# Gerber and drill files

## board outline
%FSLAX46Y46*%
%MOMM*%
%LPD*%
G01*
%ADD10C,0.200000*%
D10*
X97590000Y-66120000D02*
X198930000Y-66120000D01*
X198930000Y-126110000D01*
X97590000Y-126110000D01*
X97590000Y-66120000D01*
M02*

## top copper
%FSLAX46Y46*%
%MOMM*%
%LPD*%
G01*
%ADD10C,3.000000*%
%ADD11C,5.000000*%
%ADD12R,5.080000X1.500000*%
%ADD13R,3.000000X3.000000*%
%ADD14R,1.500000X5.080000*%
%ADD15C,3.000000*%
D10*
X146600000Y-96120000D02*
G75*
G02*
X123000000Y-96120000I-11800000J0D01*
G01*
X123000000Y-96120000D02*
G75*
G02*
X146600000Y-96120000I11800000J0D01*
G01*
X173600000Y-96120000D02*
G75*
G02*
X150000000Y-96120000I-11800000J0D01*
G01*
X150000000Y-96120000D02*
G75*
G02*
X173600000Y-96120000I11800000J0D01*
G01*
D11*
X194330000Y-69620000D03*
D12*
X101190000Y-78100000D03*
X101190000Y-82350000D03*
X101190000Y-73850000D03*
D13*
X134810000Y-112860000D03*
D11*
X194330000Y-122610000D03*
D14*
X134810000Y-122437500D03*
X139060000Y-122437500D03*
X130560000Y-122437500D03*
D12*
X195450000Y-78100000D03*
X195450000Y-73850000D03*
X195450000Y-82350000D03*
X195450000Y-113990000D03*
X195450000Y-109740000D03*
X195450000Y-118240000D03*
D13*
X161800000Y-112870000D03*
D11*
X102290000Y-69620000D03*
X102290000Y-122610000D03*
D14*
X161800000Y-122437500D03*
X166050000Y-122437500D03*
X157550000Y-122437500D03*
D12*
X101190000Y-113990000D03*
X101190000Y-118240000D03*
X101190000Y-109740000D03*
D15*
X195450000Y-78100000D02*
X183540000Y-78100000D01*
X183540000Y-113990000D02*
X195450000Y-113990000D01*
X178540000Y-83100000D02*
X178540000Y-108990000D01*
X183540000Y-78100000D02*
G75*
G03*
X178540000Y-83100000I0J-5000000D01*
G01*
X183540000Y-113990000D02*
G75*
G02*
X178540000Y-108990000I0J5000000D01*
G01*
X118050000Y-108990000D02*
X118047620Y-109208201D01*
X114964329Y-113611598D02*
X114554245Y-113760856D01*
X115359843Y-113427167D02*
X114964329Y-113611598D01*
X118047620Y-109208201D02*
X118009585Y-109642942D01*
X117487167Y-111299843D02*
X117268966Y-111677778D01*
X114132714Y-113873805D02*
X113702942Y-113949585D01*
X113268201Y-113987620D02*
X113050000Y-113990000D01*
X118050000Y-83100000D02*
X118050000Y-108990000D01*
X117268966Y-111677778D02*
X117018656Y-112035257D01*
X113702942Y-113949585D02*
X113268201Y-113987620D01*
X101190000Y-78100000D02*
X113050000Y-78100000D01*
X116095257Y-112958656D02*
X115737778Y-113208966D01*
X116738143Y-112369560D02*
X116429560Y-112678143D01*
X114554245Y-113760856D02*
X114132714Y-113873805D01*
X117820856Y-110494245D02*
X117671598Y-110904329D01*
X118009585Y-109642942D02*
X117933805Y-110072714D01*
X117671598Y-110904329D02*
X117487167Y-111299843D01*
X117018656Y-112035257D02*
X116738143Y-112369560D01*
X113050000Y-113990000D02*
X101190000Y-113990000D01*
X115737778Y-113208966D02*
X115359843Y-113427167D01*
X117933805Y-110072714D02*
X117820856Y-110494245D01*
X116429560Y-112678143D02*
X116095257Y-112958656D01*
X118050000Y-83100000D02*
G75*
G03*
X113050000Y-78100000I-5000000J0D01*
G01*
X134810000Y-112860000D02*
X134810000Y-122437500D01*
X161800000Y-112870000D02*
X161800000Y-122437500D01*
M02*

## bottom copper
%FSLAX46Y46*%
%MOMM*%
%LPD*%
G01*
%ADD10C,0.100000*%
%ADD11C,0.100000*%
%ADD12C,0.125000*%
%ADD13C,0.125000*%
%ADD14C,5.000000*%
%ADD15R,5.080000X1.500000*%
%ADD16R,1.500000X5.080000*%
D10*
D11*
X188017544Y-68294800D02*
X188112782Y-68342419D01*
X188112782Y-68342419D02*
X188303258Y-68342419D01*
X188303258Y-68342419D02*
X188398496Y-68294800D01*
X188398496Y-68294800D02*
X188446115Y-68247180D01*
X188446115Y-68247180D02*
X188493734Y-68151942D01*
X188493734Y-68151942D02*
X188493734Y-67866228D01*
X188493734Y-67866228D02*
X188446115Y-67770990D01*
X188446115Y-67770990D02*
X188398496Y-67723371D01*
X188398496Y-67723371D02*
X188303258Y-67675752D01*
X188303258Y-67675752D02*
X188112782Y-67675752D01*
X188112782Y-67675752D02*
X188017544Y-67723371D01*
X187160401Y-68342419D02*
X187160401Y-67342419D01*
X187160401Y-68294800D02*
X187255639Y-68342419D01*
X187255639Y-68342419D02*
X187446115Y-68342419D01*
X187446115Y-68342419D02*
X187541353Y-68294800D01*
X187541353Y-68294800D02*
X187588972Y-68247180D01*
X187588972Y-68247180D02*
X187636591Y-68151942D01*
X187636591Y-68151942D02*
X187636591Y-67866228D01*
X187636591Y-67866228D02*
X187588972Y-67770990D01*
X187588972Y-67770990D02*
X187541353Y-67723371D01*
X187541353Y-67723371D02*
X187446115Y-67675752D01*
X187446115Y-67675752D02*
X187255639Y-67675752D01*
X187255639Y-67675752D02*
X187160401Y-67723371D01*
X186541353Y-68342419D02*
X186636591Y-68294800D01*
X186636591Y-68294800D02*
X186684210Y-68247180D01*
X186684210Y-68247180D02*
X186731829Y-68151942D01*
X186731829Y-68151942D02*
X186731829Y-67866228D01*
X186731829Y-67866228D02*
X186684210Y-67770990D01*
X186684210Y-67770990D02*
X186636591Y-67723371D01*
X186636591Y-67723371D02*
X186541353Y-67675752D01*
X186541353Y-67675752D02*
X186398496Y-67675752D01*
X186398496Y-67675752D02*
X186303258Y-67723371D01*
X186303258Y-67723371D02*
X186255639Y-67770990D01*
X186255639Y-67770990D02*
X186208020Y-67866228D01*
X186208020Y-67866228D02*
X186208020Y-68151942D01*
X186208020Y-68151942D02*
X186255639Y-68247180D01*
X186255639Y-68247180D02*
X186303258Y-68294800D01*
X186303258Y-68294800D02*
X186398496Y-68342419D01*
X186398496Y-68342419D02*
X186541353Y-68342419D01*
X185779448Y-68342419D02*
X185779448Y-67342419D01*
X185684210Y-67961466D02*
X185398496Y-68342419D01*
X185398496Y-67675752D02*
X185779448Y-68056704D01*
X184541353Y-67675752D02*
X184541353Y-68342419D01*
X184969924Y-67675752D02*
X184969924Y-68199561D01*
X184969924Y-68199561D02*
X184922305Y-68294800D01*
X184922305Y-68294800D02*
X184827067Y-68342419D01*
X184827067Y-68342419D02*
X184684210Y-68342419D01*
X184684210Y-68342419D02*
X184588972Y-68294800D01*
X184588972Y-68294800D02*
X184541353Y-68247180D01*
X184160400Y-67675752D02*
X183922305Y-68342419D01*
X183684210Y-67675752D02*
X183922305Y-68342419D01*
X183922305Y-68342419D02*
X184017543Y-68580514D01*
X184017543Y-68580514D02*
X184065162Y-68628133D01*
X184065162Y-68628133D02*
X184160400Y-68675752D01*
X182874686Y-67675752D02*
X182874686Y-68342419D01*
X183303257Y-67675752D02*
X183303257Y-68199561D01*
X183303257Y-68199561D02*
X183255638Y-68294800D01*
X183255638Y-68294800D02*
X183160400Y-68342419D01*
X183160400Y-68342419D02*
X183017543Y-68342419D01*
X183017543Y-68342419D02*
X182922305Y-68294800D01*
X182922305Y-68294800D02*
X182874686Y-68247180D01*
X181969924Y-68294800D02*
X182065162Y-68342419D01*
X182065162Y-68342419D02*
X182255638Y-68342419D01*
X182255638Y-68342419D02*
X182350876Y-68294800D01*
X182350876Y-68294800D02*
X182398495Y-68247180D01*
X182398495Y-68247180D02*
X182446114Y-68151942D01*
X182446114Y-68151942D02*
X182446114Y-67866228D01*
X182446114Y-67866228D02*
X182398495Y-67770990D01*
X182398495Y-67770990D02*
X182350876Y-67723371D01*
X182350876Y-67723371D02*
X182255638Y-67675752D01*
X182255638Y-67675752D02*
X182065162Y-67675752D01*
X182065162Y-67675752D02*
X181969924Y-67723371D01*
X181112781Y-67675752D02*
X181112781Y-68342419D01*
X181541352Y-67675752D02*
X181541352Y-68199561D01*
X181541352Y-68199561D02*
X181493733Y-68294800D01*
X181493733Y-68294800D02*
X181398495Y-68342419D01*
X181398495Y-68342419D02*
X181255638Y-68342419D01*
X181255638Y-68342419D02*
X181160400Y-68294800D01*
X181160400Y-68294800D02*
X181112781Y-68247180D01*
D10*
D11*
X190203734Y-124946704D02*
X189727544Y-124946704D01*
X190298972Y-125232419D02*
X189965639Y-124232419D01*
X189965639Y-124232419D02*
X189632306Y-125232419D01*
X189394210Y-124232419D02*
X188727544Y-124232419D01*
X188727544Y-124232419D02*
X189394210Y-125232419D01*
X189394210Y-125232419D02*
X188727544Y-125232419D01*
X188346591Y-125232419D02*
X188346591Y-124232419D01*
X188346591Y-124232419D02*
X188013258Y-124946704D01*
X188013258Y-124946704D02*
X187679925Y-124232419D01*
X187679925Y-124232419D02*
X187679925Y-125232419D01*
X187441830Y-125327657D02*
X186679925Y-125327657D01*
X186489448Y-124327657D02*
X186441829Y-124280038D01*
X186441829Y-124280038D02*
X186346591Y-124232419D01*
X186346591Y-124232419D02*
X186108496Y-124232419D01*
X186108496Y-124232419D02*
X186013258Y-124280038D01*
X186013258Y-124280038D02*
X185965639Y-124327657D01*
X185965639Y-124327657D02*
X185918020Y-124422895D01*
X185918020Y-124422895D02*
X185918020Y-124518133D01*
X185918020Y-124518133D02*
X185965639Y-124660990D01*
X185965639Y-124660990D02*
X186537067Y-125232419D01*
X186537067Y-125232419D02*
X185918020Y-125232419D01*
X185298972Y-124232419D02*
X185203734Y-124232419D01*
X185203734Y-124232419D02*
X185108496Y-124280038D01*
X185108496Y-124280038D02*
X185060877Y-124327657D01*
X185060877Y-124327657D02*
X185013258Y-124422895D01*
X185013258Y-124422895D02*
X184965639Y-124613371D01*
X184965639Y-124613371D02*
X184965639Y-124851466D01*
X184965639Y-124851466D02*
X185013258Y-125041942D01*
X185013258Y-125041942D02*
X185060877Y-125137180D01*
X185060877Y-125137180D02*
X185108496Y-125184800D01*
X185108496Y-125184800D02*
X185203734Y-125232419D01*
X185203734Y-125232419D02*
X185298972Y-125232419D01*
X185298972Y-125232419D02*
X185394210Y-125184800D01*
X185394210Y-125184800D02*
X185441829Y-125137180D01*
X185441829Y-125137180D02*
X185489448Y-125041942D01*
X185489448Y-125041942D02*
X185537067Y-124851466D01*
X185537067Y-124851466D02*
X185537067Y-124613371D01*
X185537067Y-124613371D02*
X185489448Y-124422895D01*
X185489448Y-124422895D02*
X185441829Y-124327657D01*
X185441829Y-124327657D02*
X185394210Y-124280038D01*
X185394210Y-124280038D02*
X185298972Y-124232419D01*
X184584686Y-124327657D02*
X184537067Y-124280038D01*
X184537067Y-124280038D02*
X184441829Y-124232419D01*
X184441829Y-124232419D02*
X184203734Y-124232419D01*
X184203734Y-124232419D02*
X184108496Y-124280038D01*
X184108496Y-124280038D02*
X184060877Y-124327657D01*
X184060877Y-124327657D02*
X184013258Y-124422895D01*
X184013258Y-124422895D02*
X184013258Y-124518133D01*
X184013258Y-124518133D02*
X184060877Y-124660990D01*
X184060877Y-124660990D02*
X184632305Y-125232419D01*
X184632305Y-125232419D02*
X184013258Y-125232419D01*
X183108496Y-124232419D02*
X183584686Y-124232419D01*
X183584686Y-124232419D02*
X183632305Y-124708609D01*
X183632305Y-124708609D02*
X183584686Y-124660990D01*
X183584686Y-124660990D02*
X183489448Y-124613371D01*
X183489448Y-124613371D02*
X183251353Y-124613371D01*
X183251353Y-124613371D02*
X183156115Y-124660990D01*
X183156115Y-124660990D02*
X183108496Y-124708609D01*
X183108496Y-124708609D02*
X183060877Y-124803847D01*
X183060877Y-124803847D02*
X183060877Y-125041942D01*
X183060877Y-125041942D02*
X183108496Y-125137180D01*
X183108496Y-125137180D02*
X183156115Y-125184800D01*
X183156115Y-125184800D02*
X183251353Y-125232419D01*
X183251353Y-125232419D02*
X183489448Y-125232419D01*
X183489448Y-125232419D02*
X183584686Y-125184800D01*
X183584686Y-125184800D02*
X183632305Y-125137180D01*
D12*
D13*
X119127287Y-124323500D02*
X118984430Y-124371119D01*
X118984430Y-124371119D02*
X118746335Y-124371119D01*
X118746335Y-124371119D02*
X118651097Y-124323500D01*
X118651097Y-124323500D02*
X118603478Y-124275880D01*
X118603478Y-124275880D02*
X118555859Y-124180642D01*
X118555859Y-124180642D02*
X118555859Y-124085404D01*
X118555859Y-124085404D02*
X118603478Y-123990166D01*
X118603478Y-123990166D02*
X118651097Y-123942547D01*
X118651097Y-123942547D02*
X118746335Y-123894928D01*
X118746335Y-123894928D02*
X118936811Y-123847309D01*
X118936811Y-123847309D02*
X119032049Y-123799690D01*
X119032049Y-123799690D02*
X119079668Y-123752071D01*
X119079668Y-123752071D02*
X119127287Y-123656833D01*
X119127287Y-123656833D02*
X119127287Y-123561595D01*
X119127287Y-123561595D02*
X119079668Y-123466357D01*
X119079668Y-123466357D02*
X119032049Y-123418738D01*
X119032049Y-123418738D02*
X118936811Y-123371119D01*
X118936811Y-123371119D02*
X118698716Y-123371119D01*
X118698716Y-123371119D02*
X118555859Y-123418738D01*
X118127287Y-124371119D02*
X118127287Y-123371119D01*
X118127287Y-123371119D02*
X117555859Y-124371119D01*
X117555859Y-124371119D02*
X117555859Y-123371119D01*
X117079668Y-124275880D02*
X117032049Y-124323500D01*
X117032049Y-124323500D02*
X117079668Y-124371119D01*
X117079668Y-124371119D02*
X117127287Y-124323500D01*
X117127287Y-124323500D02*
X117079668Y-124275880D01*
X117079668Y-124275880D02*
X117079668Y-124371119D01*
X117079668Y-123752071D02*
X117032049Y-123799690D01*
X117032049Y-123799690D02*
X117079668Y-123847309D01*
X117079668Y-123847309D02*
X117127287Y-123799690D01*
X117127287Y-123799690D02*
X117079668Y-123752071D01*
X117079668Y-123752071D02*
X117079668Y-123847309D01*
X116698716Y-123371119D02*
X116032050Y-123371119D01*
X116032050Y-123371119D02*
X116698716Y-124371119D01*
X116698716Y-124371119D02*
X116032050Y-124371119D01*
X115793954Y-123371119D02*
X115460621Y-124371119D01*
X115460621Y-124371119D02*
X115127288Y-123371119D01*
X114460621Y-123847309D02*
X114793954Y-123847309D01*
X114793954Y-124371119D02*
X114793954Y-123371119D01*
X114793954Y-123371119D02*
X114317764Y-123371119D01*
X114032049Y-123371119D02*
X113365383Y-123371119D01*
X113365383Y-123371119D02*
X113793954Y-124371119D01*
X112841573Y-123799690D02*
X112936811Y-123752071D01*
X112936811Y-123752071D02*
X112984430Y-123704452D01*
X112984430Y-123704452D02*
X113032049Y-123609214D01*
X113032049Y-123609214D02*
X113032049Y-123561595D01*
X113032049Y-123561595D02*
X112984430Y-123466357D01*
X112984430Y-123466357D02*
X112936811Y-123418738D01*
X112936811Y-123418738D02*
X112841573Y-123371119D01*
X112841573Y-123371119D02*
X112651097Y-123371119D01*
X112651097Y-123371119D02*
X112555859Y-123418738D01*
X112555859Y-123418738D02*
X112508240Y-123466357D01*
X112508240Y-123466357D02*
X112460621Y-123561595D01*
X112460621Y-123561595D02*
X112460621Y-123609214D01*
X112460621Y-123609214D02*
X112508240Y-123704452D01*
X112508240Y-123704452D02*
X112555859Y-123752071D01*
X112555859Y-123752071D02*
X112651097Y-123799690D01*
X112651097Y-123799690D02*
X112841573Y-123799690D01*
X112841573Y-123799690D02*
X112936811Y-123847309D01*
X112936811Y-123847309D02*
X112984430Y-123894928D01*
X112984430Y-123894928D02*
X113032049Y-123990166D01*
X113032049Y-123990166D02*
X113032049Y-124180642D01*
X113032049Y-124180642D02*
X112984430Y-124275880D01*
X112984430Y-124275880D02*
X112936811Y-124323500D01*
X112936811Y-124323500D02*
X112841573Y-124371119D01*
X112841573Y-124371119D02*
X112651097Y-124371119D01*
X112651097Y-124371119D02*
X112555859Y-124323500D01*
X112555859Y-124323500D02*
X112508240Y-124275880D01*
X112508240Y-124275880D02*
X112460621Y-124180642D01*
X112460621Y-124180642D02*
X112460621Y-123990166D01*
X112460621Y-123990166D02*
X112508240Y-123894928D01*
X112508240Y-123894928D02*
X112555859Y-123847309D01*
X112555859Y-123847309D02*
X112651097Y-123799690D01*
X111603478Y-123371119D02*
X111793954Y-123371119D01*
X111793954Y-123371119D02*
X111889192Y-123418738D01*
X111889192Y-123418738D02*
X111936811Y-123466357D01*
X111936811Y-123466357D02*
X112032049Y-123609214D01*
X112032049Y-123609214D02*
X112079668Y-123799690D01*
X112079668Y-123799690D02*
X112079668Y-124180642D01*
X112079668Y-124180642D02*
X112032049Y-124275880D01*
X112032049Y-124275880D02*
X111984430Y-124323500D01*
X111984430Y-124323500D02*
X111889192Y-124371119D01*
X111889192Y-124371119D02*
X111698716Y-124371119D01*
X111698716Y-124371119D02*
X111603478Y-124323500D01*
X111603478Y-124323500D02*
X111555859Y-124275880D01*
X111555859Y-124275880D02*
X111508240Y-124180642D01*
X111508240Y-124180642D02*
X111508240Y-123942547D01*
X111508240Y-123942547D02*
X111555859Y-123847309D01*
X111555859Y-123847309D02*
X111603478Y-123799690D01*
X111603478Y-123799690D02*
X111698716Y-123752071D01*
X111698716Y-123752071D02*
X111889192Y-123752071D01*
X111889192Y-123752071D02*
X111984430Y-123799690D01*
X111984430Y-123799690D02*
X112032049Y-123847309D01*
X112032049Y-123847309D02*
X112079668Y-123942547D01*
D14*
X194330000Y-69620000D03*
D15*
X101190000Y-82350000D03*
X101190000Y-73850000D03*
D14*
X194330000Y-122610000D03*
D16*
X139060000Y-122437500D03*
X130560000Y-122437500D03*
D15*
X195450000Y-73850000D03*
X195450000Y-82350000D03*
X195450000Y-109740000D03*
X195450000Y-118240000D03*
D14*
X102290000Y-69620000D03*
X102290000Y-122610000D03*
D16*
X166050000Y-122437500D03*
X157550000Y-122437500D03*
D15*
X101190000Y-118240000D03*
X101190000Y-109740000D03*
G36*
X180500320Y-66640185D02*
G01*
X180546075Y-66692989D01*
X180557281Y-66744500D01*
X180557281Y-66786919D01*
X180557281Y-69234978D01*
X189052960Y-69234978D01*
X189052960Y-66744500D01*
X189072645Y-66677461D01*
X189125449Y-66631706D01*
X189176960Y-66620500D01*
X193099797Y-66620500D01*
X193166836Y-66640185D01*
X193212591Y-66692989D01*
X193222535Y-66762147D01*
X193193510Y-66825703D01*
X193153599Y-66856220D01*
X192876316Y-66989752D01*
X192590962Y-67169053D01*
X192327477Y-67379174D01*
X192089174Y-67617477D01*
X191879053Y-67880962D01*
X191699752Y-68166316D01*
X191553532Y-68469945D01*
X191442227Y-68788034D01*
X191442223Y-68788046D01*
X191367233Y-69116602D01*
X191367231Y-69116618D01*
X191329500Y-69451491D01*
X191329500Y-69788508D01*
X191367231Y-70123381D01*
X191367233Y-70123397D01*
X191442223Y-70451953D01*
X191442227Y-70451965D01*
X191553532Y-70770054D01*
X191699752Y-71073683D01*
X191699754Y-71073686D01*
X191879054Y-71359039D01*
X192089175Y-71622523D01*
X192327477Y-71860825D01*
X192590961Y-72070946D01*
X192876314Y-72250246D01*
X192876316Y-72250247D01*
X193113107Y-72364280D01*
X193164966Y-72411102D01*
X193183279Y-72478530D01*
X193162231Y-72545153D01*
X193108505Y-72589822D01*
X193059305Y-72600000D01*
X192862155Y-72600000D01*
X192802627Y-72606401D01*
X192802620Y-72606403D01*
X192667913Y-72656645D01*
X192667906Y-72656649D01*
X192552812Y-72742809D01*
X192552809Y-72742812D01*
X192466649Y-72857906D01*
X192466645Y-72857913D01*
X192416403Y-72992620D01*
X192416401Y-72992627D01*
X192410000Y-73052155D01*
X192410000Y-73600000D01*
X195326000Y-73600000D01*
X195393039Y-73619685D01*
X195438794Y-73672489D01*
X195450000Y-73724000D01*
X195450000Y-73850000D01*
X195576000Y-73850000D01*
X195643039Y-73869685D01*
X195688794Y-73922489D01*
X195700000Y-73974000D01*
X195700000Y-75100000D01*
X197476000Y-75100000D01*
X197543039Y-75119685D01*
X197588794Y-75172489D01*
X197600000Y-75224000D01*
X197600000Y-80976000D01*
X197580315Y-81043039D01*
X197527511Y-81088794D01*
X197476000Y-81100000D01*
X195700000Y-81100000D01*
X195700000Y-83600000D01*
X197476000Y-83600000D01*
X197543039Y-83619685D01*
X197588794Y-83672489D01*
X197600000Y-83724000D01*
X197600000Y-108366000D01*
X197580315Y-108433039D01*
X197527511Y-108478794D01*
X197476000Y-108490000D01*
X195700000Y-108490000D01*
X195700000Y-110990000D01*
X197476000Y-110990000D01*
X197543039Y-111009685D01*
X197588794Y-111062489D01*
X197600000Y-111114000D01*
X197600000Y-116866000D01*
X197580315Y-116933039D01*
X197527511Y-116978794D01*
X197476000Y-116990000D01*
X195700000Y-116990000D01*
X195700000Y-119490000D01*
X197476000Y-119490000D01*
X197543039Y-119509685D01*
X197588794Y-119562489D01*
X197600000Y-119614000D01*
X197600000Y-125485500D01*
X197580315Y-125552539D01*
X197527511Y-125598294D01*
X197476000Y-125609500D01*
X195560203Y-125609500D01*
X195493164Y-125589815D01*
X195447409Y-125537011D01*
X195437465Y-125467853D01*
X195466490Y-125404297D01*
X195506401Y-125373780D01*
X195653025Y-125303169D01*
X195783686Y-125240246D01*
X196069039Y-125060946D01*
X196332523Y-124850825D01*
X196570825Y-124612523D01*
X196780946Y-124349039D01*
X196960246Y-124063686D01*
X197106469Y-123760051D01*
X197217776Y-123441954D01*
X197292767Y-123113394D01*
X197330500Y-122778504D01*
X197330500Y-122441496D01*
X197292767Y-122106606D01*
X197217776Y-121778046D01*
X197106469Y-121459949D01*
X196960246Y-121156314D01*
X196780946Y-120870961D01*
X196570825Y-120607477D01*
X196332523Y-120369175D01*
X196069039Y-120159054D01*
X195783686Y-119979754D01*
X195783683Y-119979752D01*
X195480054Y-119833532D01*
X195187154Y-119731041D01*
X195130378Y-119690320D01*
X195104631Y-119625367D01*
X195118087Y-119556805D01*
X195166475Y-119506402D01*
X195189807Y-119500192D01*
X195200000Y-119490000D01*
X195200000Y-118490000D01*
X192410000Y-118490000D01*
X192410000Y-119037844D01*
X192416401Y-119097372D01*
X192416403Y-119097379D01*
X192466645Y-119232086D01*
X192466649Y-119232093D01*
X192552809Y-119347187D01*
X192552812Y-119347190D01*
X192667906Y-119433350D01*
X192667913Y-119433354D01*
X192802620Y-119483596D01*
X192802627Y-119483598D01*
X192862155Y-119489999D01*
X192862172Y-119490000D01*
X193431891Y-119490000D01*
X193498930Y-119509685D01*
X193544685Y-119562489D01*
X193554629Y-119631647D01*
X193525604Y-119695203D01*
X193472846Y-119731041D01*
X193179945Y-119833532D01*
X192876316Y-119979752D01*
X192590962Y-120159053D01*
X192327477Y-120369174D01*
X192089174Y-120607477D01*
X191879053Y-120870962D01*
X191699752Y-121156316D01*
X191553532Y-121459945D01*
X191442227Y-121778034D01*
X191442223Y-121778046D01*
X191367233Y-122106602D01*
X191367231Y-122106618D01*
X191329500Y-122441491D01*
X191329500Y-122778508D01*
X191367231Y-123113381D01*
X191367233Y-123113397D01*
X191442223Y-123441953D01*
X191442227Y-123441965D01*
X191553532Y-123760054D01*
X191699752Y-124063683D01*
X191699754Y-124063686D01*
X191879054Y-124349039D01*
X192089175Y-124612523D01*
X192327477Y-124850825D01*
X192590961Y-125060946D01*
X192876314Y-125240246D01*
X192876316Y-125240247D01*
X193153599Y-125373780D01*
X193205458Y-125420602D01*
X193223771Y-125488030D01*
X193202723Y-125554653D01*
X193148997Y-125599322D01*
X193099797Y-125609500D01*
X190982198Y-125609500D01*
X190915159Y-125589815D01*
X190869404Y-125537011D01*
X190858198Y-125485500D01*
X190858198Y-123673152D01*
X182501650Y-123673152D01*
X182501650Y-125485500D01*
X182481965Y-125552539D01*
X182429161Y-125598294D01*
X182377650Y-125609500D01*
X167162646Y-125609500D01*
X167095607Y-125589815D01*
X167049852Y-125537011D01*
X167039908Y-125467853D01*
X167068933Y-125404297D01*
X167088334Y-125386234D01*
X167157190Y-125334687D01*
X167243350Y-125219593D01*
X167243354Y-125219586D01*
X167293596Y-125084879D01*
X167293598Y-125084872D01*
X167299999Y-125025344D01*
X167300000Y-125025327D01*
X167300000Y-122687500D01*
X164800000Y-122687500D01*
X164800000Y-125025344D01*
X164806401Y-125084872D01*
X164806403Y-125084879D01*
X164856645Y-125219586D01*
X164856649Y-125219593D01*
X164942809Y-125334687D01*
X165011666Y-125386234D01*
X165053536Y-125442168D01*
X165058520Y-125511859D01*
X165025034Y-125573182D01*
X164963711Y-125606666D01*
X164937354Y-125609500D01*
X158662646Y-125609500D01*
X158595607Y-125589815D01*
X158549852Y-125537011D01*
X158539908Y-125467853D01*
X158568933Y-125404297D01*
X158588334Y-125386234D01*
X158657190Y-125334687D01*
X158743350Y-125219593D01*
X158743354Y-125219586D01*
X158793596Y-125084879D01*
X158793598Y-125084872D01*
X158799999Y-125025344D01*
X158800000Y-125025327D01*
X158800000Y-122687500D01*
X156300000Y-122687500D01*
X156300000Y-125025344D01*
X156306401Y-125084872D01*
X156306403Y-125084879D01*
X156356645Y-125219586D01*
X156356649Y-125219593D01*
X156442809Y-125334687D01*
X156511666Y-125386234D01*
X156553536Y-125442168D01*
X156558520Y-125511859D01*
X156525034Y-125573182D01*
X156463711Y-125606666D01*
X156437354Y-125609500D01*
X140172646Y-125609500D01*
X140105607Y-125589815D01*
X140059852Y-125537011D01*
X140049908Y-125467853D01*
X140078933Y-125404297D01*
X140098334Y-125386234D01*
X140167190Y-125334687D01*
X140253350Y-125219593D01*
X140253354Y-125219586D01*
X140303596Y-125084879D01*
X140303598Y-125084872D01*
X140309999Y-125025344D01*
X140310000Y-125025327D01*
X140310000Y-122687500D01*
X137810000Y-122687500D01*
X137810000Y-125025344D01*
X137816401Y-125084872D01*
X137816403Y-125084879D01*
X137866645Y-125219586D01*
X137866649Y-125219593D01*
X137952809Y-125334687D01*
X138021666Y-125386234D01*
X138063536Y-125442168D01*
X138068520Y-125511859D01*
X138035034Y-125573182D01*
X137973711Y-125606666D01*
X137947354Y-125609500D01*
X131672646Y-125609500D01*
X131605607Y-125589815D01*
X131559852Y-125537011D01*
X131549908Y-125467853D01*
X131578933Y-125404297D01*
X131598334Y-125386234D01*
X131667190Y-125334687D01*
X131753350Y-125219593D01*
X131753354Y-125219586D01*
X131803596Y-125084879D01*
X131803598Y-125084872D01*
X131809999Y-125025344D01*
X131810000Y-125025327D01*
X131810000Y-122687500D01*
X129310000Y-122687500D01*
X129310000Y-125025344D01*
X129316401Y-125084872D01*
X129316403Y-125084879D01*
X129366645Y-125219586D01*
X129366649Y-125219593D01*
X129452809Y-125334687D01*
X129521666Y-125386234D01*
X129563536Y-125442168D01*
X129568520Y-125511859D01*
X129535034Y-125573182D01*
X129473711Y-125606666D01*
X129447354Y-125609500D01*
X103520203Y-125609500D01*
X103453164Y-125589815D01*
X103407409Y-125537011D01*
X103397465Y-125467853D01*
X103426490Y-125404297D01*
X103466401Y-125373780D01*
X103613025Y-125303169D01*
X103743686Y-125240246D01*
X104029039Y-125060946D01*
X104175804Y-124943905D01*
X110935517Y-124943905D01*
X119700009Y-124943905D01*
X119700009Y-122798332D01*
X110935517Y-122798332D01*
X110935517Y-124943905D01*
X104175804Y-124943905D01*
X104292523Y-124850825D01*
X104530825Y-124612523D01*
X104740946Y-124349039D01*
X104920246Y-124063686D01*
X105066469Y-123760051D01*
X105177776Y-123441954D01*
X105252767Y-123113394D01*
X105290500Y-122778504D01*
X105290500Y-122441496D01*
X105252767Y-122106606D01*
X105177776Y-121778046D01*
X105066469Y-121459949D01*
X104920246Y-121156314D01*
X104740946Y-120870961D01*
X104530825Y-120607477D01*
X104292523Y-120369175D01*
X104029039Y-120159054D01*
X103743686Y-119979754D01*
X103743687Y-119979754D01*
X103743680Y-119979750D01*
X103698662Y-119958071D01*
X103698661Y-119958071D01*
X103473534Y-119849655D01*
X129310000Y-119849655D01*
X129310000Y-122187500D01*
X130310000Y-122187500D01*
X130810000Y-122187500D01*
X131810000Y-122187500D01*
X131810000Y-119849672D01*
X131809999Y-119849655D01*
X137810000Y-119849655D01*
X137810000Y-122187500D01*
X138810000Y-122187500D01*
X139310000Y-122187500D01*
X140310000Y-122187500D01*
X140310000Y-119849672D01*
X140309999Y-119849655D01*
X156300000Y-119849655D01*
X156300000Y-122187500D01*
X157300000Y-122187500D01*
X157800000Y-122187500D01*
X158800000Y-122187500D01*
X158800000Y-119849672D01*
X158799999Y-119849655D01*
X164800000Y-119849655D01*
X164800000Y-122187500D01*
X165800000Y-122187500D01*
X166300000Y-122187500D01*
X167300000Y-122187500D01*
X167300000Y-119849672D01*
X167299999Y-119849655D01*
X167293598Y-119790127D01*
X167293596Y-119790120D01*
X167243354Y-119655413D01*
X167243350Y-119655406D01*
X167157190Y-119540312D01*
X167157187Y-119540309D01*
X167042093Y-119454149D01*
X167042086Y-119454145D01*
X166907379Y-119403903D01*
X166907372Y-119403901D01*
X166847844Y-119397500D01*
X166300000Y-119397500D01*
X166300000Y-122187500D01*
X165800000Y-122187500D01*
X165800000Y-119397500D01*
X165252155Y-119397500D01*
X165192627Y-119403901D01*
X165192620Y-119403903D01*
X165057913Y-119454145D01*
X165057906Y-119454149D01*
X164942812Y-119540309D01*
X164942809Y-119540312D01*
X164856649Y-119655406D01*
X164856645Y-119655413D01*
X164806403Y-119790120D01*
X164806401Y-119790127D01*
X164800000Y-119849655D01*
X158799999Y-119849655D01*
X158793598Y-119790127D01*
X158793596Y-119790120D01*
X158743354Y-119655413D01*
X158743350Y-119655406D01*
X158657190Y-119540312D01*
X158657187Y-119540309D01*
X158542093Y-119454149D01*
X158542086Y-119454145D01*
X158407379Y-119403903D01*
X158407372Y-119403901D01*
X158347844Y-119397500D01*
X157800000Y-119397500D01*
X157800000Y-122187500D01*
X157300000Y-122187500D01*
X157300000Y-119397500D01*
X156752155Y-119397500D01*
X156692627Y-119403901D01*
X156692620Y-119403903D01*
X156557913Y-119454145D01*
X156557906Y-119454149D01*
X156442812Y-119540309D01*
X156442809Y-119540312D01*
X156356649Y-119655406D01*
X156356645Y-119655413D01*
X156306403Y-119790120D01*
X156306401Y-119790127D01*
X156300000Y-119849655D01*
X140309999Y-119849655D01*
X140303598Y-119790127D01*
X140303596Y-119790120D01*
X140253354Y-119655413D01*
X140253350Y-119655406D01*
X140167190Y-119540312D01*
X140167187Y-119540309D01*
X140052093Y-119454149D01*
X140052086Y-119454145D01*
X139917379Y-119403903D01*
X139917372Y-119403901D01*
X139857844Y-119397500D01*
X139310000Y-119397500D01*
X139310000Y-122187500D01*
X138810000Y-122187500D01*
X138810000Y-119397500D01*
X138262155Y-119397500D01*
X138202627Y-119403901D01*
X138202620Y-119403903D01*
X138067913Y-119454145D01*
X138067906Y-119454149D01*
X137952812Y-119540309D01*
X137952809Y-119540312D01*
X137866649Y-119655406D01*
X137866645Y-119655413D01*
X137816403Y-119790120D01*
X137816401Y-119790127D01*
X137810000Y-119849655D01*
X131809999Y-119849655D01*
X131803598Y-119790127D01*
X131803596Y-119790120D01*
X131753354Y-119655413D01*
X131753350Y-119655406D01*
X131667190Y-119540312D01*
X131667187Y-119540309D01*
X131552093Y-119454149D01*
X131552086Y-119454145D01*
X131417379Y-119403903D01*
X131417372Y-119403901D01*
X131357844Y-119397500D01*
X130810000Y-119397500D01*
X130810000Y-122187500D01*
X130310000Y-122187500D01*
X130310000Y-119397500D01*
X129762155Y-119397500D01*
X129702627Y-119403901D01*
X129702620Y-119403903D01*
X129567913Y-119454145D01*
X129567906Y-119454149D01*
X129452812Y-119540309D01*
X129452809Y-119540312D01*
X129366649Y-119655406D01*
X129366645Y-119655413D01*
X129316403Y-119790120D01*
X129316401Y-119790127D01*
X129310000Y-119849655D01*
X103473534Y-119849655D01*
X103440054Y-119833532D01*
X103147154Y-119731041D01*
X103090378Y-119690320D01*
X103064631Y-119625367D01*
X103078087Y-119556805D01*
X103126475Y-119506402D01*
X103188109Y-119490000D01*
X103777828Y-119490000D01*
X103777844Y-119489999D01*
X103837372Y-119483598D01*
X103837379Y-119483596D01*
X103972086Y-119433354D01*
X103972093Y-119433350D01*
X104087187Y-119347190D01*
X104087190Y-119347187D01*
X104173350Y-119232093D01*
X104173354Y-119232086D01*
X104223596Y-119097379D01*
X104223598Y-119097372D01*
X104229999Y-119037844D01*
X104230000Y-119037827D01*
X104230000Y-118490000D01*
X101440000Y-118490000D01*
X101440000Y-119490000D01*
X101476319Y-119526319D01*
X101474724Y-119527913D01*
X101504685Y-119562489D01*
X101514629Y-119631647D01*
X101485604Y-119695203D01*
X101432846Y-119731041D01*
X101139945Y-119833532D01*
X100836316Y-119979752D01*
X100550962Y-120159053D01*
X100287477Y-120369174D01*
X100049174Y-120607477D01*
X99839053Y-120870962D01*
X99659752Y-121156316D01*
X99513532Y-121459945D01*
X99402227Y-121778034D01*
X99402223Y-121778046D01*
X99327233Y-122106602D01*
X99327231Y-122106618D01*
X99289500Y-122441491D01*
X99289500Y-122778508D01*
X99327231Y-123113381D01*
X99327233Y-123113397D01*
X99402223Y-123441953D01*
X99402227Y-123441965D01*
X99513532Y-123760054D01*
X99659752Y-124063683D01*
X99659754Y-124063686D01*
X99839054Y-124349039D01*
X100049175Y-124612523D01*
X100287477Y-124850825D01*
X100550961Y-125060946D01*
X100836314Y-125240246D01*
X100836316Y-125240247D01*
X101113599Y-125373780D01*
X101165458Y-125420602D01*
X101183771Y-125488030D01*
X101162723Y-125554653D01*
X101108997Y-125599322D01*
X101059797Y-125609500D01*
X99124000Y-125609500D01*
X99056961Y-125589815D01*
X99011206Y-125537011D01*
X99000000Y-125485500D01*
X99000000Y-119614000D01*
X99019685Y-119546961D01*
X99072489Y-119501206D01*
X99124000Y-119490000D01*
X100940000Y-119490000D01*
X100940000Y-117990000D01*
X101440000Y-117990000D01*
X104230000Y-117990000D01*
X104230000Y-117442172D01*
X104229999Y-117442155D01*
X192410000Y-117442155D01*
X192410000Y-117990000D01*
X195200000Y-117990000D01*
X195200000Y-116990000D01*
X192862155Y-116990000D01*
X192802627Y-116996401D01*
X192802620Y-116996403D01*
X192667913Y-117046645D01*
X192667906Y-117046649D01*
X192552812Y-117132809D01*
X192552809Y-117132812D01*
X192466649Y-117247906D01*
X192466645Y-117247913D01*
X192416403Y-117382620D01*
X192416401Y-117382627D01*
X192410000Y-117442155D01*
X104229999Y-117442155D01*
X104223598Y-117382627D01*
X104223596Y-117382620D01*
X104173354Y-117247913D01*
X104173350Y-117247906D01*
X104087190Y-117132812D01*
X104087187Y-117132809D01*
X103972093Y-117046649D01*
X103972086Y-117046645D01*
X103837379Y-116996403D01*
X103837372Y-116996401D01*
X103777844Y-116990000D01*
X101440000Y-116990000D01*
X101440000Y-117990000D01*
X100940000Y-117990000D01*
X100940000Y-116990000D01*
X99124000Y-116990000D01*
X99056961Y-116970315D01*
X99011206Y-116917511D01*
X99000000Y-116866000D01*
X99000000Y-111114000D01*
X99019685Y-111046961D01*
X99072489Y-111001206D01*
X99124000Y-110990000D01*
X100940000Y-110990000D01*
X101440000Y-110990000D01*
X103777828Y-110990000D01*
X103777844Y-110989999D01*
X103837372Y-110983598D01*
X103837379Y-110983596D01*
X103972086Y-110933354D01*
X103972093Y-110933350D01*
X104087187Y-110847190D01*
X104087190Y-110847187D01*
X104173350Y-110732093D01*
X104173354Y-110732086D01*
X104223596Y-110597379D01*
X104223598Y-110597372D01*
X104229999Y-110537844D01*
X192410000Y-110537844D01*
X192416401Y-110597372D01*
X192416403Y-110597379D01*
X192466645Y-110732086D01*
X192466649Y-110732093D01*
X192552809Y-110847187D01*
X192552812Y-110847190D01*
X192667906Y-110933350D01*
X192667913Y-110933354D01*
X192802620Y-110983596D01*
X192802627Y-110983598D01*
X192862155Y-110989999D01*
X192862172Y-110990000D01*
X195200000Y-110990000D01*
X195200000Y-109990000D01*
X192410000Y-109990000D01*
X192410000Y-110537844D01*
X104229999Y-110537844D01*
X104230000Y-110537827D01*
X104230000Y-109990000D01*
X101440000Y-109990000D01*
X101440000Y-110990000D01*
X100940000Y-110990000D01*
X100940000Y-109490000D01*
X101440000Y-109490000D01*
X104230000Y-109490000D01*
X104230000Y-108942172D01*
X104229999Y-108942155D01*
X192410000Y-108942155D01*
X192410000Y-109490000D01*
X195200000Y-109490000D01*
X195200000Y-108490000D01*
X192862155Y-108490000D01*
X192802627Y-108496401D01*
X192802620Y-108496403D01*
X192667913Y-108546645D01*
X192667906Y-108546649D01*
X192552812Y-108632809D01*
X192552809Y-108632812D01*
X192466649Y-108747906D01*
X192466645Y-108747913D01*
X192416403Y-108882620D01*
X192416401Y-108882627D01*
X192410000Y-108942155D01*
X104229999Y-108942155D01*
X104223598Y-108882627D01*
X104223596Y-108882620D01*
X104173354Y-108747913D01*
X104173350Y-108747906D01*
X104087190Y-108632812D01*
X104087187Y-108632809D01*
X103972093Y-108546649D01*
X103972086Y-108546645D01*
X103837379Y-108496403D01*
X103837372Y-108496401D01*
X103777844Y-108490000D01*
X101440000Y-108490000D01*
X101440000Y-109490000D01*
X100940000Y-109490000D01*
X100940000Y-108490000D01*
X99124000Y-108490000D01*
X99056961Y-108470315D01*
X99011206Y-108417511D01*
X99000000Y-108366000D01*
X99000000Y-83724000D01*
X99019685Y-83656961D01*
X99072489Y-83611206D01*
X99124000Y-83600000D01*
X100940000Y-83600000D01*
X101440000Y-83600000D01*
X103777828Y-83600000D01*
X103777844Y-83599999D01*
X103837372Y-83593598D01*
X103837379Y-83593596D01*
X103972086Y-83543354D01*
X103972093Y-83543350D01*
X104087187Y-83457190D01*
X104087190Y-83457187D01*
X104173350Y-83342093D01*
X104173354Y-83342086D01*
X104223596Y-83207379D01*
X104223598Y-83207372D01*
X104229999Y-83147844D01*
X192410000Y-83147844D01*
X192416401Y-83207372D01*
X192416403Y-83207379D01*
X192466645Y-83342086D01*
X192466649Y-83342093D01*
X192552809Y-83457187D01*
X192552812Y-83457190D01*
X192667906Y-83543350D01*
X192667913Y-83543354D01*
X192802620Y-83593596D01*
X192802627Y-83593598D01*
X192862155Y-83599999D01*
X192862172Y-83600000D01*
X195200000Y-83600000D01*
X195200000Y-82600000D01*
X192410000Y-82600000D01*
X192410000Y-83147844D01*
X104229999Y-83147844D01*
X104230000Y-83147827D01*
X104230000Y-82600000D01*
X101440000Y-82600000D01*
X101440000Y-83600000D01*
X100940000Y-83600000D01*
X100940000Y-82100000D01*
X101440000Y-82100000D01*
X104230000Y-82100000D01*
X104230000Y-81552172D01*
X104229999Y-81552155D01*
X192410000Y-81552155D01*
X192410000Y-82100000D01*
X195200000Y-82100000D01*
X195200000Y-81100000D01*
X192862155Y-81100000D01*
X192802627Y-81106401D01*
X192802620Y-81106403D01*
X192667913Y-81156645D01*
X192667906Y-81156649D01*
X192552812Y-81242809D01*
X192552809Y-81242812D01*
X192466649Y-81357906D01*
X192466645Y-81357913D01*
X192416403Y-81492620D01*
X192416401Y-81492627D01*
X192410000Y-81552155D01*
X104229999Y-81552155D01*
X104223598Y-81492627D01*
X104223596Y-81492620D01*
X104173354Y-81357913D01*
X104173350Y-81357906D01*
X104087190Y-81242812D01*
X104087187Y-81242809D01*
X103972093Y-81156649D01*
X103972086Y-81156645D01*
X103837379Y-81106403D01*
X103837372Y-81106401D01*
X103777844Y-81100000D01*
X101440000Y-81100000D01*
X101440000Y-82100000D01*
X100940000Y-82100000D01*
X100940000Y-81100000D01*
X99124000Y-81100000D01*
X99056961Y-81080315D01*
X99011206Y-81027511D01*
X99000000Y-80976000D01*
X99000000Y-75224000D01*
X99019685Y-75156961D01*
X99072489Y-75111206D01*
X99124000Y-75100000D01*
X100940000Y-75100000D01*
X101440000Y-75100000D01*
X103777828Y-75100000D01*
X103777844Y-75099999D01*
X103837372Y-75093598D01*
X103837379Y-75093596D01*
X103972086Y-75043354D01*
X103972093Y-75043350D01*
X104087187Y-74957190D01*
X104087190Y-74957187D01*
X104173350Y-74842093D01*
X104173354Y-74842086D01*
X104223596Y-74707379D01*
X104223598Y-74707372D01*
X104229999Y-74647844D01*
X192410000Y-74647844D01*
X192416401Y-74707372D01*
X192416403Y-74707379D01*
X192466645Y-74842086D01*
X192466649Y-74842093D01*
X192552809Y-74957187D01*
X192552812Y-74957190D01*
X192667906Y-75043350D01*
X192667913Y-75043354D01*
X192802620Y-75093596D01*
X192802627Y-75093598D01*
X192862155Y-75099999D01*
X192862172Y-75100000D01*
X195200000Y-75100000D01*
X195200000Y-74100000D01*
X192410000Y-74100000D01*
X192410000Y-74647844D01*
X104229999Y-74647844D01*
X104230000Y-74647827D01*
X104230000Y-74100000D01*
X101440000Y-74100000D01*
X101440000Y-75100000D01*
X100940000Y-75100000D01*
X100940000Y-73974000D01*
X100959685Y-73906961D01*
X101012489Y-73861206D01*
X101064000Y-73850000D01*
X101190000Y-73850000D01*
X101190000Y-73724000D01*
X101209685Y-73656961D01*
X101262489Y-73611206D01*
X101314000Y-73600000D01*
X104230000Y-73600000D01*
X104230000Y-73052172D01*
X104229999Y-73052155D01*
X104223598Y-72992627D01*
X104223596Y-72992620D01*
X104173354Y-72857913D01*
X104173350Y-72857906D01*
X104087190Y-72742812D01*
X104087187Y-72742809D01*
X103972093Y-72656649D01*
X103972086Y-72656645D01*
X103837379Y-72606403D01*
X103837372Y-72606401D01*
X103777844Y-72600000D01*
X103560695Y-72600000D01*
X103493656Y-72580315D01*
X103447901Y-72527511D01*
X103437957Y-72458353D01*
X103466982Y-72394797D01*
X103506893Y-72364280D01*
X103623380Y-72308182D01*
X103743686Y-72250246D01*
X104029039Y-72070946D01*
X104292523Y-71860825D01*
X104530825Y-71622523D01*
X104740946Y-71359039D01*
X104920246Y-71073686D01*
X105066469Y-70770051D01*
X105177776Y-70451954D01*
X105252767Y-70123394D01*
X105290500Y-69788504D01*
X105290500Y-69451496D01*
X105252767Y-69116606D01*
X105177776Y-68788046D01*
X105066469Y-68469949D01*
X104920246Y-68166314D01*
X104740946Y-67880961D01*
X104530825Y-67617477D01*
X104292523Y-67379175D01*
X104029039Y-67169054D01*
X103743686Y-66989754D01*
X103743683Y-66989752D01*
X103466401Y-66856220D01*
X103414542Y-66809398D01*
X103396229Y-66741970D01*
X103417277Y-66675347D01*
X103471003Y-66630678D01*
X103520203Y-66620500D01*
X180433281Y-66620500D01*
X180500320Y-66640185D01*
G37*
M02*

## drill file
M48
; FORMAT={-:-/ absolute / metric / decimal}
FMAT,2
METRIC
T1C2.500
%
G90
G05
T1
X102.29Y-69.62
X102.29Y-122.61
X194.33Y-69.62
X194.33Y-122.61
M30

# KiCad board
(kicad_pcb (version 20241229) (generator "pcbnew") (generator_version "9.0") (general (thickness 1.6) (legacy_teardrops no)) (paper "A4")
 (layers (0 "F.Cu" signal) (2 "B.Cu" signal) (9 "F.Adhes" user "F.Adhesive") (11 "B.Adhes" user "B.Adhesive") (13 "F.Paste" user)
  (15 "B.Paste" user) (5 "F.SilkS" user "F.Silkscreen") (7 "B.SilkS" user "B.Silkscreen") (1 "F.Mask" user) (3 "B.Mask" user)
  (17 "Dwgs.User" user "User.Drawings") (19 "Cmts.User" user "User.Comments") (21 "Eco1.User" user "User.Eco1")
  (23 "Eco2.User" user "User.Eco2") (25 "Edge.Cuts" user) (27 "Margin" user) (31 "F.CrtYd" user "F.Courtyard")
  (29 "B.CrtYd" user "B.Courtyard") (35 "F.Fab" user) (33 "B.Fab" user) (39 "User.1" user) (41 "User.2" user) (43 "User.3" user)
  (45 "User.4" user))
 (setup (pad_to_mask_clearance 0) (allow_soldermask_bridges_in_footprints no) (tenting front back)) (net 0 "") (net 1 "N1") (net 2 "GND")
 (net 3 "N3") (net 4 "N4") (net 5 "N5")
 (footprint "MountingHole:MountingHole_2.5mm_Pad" (layer "F.Cu") (at 194.33 69.62)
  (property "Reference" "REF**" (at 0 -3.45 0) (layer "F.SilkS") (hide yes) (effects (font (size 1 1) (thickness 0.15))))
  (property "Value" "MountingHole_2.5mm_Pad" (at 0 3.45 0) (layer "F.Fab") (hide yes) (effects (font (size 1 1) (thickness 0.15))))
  (pad "1" thru_hole circle (at 0 0) (size 5 5) (drill 2.5) (layers "*.Cu" "*.Mask") (remove_unused_layers no) (zone_connect 2)))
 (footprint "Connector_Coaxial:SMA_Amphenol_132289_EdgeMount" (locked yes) (layer "F.Cu") (at 101.19 78.1 180)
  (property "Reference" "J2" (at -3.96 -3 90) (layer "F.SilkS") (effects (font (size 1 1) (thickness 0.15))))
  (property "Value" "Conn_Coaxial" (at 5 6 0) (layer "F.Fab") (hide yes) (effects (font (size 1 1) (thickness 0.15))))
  (pad "1" smd rect (at 0 0 270) (size 1.5 5.08) (layers "F.Cu" "F.Mask" "F.Paste") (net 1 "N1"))
  (pad "2" smd rect (at 0 -4.25 270) (size 1.5 5.08) (layers "F.Cu" "F.Mask" "F.Paste") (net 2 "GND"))
  (pad "2" smd rect (at 0 -4.25 270) (size 1.5 5.08) (layers "B.Cu" "B.Mask" "B.Paste") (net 2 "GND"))
  (pad "2" smd rect (at 0 4.25 270) (size 1.5 5.08) (layers "F.Cu" "F.Mask" "F.Paste") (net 2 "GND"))
  (pad "2" smd rect (at 0 4.25 270) (size 1.5 5.08) (layers "B.Cu" "B.Mask" "B.Paste") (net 2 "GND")))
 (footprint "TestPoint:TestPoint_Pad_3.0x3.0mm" (layer "F.Cu") (at 134.81 112.86 90)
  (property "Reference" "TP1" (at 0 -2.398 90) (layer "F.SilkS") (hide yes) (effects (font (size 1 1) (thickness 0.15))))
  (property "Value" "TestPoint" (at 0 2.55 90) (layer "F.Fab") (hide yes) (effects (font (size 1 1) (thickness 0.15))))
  (pad "1" smd rect (at 0 0 90) (size 3 3) (layers "F.Cu" "F.Mask") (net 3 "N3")))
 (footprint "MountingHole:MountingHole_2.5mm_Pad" (layer "F.Cu") (at 194.33 122.61)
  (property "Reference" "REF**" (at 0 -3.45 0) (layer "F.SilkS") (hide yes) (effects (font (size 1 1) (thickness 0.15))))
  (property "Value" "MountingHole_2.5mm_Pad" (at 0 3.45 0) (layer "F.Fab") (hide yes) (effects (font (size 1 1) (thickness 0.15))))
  (pad "1" thru_hole circle (at 0 0) (size 5 5) (drill 2.5) (layers "*.Cu" "*.Mask") (remove_unused_layers no) (zone_connect 2)))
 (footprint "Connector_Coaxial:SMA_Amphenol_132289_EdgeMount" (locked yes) (layer "F.Cu") (at 134.81 122.4375 -90)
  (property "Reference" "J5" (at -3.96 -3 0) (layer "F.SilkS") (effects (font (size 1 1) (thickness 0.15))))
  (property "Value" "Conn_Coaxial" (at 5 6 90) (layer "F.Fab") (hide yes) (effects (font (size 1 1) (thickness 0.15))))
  (pad "1" smd rect (at 0 0) (size 1.5 5.08) (layers "F.Cu" "F.Mask" "F.Paste") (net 3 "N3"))
  (pad "2" smd rect (at 0 -4.25) (size 1.5 5.08) (layers "F.Cu" "F.Mask" "F.Paste") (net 2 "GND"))
  (pad "2" smd rect (at 0 -4.25) (size 1.5 5.08) (layers "B.Cu" "B.Mask" "B.Paste") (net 2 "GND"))
  (pad "2" smd rect (at 0 4.25) (size 1.5 5.08) (layers "F.Cu" "F.Mask" "F.Paste") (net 2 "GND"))
  (pad "2" smd rect (at 0 4.25) (size 1.5 5.08) (layers "B.Cu" "B.Mask" "B.Paste") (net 2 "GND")))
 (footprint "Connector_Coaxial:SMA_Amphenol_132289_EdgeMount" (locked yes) (layer "F.Cu") (at 195.45 78.1)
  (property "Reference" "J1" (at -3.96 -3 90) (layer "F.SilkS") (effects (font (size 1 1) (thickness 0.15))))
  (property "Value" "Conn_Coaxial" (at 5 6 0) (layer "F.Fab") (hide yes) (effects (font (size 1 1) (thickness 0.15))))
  (pad "1" smd rect (at 0 0 90) (size 1.5 5.08) (layers "F.Cu" "F.Mask" "F.Paste") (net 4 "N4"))
  (pad "2" smd rect (at 0 -4.25 90) (size 1.5 5.08) (layers "F.Cu" "F.Mask" "F.Paste") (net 2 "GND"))
  (pad "2" smd rect (at 0 -4.25 90) (size 1.5 5.08) (layers "B.Cu" "B.Mask" "B.Paste") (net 2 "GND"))
  (pad "2" smd rect (at 0 4.25 90) (size 1.5 5.08) (layers "F.Cu" "F.Mask" "F.Paste") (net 2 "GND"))
  (pad "2" smd rect (at 0 4.25 90) (size 1.5 5.08) (layers "B.Cu" "B.Mask" "B.Paste") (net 2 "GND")))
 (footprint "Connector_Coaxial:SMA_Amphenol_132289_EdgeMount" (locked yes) (layer "F.Cu") (at 195.45 113.99)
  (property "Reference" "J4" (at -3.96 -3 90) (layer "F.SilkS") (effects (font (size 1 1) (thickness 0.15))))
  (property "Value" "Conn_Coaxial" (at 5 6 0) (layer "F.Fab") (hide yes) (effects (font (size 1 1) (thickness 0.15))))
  (pad "1" smd rect (at 0 0 90) (size 1.5 5.08) (layers "F.Cu" "F.Mask" "F.Paste") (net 4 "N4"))
  (pad "2" smd rect (at 0 -4.25 90) (size 1.5 5.08) (layers "F.Cu" "F.Mask" "F.Paste") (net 2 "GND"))
  (pad "2" smd rect (at 0 -4.25 90) (size 1.5 5.08) (layers "B.Cu" "B.Mask" "B.Paste") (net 2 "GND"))
  (pad "2" smd rect (at 0 4.25 90) (size 1.5 5.08) (layers "F.Cu" "F.Mask" "F.Paste") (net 2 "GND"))
  (pad "2" smd rect (at 0 4.25 90) (size 1.5 5.08) (layers "B.Cu" "B.Mask" "B.Paste") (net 2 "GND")))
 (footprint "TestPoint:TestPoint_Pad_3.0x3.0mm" (layer "F.Cu") (at 161.8 112.87 90)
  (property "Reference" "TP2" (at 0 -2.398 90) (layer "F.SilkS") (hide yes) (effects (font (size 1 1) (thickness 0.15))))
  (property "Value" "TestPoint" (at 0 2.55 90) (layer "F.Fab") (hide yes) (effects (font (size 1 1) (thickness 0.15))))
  (pad "1" smd rect (at 0 0 90) (size 3 3) (layers "F.Cu" "F.Mask") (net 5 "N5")))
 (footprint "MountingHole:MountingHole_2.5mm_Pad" (layer "F.Cu") (at 102.29 69.62)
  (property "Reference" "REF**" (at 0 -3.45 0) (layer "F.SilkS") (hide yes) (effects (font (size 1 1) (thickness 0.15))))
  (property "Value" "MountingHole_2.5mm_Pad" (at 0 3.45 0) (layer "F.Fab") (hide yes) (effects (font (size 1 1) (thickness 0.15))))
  (pad "1" thru_hole circle (at 0 0) (size 5 5) (drill 2.5) (layers "*.Cu" "*.Mask") (remove_unused_layers no) (zone_connect 2)))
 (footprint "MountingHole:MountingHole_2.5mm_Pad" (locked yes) (layer "F.Cu") (at 102.29 122.61)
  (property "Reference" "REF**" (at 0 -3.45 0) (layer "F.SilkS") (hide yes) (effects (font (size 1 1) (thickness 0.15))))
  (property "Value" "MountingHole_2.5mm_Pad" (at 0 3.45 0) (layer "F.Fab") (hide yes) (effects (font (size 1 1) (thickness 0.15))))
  (pad "1" thru_hole circle (at 0 0) (size 5 5) (drill 2.5) (layers "*.Cu" "*.Mask") (remove_unused_layers no) (zone_connect 2)))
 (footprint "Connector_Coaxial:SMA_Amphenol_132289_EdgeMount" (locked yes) (layer "F.Cu") (at 161.8 122.4375 -90)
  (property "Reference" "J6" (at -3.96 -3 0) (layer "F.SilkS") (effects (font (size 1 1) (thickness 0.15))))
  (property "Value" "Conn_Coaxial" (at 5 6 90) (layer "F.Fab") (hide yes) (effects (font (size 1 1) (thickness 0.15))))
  (pad "1" smd rect (at 0 0) (size 1.5 5.08) (layers "F.Cu" "F.Mask" "F.Paste") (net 5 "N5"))
  (pad "2" smd rect (at 0 -4.25) (size 1.5 5.08) (layers "F.Cu" "F.Mask" "F.Paste") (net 2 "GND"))
  (pad "2" smd rect (at 0 -4.25) (size 1.5 5.08) (layers "B.Cu" "B.Mask" "B.Paste") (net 2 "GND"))
  (pad "2" smd rect (at 0 4.25) (size 1.5 5.08) (layers "F.Cu" "F.Mask" "F.Paste") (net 2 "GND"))
  (pad "2" smd rect (at 0 4.25) (size 1.5 5.08) (layers "B.Cu" "B.Mask" "B.Paste") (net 2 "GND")))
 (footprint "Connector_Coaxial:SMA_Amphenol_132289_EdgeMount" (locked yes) (layer "F.Cu") (at 101.19 113.99 180)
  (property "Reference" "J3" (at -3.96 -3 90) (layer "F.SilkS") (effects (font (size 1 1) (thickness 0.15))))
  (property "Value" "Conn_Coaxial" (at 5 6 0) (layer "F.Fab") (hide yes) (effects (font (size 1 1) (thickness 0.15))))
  (pad "1" smd rect (at 0 0 270) (size 1.5 5.08) (layers "F.Cu" "F.Mask" "F.Paste") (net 1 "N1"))
  (pad "2" smd rect (at 0 -4.25 270) (size 1.5 5.08) (layers "F.Cu" "F.Mask" "F.Paste") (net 2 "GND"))
  (pad "2" smd rect (at 0 -4.25 270) (size 1.5 5.08) (layers "B.Cu" "B.Mask" "B.Paste") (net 2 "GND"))
  (pad "2" smd rect (at 0 4.25 270) (size 1.5 5.08) (layers "F.Cu" "F.Mask" "F.Paste") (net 2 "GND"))
  (pad "2" smd rect (at 0 4.25 270) (size 1.5 5.08) (layers "B.Cu" "B.Mask" "B.Paste") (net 2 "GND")))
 (gr_circle (center 134.8 96.12) (end 146.6 96.12) (stroke (width 3) (type solid)) (fill no) (locked yes) (layer "F.Cu"))
 (gr_circle (center 161.8 96.12) (end 173.6 96.12) (stroke (width 3) (type solid)) (fill no) (locked yes) (layer "F.Cu"))
 (gr_rect (start 97.59 66.12) (end 198.93 126.11) (stroke (width 0.2) (type solid)) (fill no) (layer "Edge.Cuts"))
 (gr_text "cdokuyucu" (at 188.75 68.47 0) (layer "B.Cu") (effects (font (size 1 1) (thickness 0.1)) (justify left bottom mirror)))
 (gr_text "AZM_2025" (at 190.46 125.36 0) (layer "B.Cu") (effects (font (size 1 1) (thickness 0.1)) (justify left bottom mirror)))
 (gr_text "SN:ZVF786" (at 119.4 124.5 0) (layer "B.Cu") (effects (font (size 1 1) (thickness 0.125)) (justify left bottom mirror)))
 (segment (start 195.45 78.1) (end 183.54 78.1) (width 3) (layer "F.Cu") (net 4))
 (segment (start 183.54 113.99) (end 195.45 113.99) (width 3) (layer "F.Cu") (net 4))
 (segment (start 178.54 83.1) (end 178.54 108.99) (width 3) (layer "F.Cu") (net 4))
 (arc (start 183.54 78.1) (mid 180.004466 79.564466) (end 178.54 83.1) (width 3) (layer "F.Cu") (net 4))
 (arc (start 183.54 113.99) (mid 180.004466 112.525534) (end 178.54 108.99) (width 3) (layer "F.Cu") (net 4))
 (segment (start 118.05 108.99) (end 118.04762 109.208201) (width 3) (layer "F.Cu") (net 1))
 (segment (start 114.964329 113.611598) (end 114.554245 113.760856) (width 3) (layer "F.Cu") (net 1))
 (segment (start 115.359843 113.427167) (end 114.964329 113.611598) (width 3) (layer "F.Cu") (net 1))
 (segment (start 118.04762 109.208201) (end 118.009585 109.642942) (width 3) (layer "F.Cu") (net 1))
 (segment (start 117.487167 111.299843) (end 117.268966 111.677778) (width 3) (layer "F.Cu") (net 1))
 (segment (start 114.132714 113.873805) (end 113.702942 113.949585) (width 3) (layer "F.Cu") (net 1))
 (segment (start 113.268201 113.98762) (end 113.05 113.99) (width 3) (layer "F.Cu") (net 1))
 (segment (start 118.05 83.1) (end 118.05 108.99) (width 3) (layer "F.Cu") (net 1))
 (segment (start 117.268966 111.677778) (end 117.018656 112.035257) (width 3) (layer "F.Cu") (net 1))
 (segment (start 113.702942 113.949585) (end 113.268201 113.98762) (width 3) (layer "F.Cu") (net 1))
 (segment (start 101.19 78.1) (end 113.05 78.1) (width 3) (layer "F.Cu") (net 1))
 (segment (start 116.095257 112.958656) (end 115.737778 113.208966) (width 3) (layer "F.Cu") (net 1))
 (segment (start 116.738143 112.36956) (end 116.42956 112.678143) (width 3) (layer "F.Cu") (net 1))
 (segment (start 114.554245 113.760856) (end 114.132714 113.873805) (width 3) (layer "F.Cu") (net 1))
 (segment (start 117.820856 110.494245) (end 117.671598 110.904329) (width 3) (layer "F.Cu") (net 1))
 (segment (start 118.009585 109.642942) (end 117.933805 110.072714) (width 3) (layer "F.Cu") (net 1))
 (segment (start 117.671598 110.904329) (end 117.487167 111.299843) (width 3) (layer "F.Cu") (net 1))
 (segment (start 117.018656 112.035257) (end 116.738143 112.36956) (width 3) (layer "F.Cu") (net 1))
 (segment (start 113.05 113.99) (end 101.19 113.99) (width 3) (layer "F.Cu") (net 1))
 (segment (start 115.737778 113.208966) (end 115.359843 113.427167) (width 3) (layer "F.Cu") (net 1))
 (segment (start 117.933805 110.072714) (end 117.820856 110.494245) (width 3) (layer "F.Cu") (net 1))
 (segment (start 116.42956 112.678143) (end 116.095257 112.958656) (width 3) (layer "F.Cu") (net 1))
 (arc (start 118.05 83.1) (mid 116.585534 79.564466) (end 113.05 78.1) (width 3) (layer "F.Cu") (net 1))
 (segment (start 134.81 112.86) (end 134.81 122.4375) (width 3) (layer "F.Cu") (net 3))
 (segment (start 161.8 112.87) (end 161.8 122.4375) (width 3) (layer "F.Cu") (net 5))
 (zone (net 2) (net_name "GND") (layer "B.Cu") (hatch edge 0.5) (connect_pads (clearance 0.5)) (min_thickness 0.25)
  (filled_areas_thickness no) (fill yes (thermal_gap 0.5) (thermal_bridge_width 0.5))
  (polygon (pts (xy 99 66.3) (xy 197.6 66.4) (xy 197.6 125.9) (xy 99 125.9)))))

